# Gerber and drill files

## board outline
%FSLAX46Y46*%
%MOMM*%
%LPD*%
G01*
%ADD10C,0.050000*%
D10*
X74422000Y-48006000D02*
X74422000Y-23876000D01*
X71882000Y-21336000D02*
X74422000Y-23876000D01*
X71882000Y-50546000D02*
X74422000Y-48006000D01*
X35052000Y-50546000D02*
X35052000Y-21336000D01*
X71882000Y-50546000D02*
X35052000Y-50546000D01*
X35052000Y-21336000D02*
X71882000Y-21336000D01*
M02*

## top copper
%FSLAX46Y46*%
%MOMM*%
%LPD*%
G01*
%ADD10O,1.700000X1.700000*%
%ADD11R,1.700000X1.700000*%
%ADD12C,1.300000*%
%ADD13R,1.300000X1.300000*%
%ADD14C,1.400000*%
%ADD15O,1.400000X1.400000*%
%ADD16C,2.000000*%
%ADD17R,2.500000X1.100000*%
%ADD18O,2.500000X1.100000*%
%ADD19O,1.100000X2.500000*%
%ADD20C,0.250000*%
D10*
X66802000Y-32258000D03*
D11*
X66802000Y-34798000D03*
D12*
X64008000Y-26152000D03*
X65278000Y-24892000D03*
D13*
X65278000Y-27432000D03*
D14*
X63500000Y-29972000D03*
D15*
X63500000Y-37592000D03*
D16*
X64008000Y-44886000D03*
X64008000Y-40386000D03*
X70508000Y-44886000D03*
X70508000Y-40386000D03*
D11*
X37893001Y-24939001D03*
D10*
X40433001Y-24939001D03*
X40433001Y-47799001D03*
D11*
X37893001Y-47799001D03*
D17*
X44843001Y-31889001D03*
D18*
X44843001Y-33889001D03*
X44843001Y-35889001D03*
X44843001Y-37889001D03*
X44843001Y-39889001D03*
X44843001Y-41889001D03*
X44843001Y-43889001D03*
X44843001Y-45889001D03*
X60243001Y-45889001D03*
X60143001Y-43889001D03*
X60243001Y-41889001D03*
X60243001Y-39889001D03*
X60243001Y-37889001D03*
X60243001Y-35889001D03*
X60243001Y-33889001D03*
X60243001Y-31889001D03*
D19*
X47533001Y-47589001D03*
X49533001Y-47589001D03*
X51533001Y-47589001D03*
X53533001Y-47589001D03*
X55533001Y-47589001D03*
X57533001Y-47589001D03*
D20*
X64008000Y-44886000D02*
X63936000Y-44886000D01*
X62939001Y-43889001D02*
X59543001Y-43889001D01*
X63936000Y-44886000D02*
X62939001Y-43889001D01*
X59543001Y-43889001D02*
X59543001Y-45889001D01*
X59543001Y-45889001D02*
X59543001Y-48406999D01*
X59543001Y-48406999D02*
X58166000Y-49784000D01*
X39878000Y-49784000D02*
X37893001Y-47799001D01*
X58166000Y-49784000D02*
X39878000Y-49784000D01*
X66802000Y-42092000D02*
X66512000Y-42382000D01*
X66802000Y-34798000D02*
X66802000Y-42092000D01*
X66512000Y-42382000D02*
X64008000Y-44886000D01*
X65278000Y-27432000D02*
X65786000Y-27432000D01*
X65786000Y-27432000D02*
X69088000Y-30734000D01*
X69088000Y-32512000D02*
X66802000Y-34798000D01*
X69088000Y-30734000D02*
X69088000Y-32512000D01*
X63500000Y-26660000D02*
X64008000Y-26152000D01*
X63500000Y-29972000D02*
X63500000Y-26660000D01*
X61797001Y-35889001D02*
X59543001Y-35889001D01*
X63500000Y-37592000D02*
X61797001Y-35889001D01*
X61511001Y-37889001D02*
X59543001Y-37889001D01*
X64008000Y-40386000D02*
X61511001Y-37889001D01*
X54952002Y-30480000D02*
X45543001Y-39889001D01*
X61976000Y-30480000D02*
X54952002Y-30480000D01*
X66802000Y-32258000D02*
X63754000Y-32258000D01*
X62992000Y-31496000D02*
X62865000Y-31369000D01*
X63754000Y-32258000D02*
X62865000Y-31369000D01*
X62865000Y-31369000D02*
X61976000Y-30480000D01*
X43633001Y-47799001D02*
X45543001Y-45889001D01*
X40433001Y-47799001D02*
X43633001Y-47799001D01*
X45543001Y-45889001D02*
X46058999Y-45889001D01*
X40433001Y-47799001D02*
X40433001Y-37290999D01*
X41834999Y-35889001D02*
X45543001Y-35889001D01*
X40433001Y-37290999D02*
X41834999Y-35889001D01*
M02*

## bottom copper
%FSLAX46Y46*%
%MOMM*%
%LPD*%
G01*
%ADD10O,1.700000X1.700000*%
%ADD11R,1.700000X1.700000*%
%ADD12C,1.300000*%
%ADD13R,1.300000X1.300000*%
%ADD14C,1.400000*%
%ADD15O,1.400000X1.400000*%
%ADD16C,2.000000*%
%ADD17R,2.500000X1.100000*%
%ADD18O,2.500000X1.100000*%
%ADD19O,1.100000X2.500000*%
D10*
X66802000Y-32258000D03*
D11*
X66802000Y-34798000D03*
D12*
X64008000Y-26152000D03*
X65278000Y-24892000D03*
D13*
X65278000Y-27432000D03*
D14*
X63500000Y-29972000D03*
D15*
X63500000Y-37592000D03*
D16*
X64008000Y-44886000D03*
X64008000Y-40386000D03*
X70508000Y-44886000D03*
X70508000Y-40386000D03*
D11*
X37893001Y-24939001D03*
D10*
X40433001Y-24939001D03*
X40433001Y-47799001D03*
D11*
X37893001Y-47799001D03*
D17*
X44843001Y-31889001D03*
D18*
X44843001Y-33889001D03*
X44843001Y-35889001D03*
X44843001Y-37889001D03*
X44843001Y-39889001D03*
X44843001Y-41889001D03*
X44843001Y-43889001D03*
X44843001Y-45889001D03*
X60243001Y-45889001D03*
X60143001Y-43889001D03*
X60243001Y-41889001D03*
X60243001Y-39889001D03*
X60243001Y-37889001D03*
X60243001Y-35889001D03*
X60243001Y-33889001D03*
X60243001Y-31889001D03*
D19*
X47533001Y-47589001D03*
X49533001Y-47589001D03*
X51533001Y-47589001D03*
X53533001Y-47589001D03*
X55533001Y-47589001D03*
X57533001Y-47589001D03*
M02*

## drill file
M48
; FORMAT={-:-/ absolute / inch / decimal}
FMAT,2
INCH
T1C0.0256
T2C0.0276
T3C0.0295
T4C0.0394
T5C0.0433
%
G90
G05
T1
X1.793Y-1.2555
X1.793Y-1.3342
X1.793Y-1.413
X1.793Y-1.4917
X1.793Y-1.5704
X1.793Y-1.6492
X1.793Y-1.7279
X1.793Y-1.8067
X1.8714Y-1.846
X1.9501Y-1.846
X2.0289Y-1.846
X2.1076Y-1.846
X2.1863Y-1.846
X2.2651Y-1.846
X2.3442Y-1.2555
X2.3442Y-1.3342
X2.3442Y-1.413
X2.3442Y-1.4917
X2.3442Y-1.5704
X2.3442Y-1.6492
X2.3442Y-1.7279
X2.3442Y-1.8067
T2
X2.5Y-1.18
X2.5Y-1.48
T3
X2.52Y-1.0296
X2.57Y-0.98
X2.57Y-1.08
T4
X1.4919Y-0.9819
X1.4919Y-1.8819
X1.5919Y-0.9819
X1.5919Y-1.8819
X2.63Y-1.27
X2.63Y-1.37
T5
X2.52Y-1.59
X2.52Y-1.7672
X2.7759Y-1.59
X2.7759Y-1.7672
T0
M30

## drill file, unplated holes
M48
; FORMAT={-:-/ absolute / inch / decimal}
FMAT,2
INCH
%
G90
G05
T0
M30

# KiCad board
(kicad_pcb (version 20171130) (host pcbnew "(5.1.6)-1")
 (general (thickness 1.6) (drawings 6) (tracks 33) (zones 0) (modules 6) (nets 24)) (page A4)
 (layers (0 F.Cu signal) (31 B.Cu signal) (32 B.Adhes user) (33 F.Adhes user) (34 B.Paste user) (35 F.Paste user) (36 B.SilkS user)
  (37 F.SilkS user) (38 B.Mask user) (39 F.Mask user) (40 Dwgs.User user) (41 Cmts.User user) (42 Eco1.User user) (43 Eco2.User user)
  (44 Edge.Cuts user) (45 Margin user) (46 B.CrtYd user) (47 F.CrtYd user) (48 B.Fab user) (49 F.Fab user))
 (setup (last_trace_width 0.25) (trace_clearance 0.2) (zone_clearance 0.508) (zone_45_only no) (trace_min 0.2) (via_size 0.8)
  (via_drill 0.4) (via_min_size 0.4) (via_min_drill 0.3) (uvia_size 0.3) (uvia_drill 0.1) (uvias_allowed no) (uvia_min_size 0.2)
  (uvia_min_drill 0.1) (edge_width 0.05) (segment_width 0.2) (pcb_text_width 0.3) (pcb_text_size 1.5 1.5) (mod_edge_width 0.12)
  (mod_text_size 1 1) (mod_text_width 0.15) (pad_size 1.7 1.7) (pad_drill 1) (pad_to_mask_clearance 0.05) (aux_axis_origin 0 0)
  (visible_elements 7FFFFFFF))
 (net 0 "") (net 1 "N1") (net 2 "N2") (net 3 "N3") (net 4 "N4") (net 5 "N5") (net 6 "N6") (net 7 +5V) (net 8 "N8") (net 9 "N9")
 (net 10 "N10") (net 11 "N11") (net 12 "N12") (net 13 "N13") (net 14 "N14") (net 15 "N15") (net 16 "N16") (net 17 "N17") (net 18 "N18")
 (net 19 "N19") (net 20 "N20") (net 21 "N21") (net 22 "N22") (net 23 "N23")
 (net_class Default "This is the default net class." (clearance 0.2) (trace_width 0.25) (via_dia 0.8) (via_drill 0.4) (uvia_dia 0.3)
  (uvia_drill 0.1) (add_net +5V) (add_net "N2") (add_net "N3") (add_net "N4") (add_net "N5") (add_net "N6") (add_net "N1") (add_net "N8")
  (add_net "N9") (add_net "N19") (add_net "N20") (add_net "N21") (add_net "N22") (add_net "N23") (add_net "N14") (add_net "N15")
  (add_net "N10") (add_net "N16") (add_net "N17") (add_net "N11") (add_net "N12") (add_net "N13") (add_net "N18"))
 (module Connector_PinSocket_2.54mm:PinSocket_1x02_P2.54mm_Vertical (layer F.Cu) (at 66.802 34.798 180)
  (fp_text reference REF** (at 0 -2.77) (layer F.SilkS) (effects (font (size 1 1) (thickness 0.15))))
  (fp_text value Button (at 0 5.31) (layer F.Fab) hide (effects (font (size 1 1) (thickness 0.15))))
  (pad 2 thru_hole oval (at 0 2.54 180) (size 1.7 1.7) (drill 1) (layers *.Cu *.Mask) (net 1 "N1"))
  (pad 1 thru_hole rect (at 0 0 180) (size 1.7 1.7) (drill 1) (layers *.Cu *.Mask) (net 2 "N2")))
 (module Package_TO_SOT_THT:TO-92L (layer F.Cu) (at 65.278 27.432 90)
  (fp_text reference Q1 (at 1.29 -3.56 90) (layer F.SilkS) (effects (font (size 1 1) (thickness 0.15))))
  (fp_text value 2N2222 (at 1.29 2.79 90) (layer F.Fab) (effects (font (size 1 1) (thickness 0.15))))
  (pad 2 thru_hole circle (at 1.28 -1.27 180) (size 1.3 1.3) (drill 0.75) (layers *.Cu *.Mask) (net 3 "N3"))
  (pad 3 thru_hole circle (at 2.54 0 180) (size 1.3 1.3) (drill 0.75) (layers *.Cu *.Mask) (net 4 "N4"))
  (pad 1 thru_hole rect (at 0 0 180) (size 1.3 1.3) (drill 0.75) (layers *.Cu *.Mask) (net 2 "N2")))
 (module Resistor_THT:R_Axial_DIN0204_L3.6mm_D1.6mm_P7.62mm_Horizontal (layer F.Cu) (at 63.5 29.972 270)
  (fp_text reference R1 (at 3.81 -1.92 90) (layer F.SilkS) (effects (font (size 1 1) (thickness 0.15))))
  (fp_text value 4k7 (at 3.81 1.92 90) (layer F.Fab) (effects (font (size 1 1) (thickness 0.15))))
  (pad 1 thru_hole circle (at 0 0 270) (size 1.4 1.4) (drill 0.7) (layers *.Cu *.Mask) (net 3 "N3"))
  (pad 2 thru_hole oval (at 7.62 0 270) (size 1.4 1.4) (drill 0.7) (layers *.Cu *.Mask) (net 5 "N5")))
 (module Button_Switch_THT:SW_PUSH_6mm (layer F.Cu) (at 64.008 40.386)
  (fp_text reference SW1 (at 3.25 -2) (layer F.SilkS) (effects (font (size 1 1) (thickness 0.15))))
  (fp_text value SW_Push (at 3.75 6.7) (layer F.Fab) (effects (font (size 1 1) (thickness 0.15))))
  (pad 2 thru_hole circle (at 0 4.5 90) (size 2 2) (drill 1.1) (layers *.Cu *.Mask) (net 2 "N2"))
  (pad 1 thru_hole circle (at 0 0 90) (size 2 2) (drill 1.1) (layers *.Cu *.Mask) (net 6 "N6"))
  (pad 2 thru_hole circle (at 6.5 4.5 90) (size 2 2) (drill 1.1) (layers *.Cu *.Mask))
  (pad 1 thru_hole circle (at 6.5 0 90) (size 2 2) (drill 1.1) (layers *.Cu *.Mask)))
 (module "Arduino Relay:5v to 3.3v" (layer F.Cu) (at 39.163001 36.369001)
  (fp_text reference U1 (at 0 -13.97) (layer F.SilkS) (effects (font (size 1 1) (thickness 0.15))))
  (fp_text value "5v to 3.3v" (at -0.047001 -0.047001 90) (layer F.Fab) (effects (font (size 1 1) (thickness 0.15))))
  (pad 1 thru_hole rect (at -1.27 -11.43) (size 1.7 1.7) (drill 1) (layers *.Cu *.Mask))
  (pad 2 thru_hole oval (at 1.27 -11.43) (size 1.7 1.7) (drill 1) (layers *.Cu *.Mask) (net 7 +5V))
  (pad 3 thru_hole oval (at 1.27 11.43) (size 1.7 1.7) (drill 1) (layers *.Cu *.Mask) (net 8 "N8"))
  (pad 1 thru_hole rect (at -1.27 11.43) (size 1.7 1.7) (drill 1) (layers *.Cu *.Mask) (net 2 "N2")))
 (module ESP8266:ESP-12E (layer F.Cu) (at 45.543001 31.889001)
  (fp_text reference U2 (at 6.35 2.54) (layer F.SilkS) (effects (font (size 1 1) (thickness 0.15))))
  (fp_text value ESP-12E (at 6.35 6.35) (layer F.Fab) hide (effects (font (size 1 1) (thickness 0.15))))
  (pad 1 thru_hole rect (at 0 0) (size 2.5 1.1) (drill 0.65 (offset -0.7 0)) (layers *.Cu *.Mask F.SilkS) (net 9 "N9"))
  (pad 2 thru_hole oval (at 0 2) (size 2.5 1.1) (drill 0.65 (offset -0.7 0)) (layers *.Cu *.Mask F.SilkS) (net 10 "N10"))
  (pad 3 thru_hole oval (at 0 4) (size 2.5 1.1) (drill 0.65 (offset -0.7 0)) (layers *.Cu *.Mask F.SilkS) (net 8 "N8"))
  (pad 4 thru_hole oval (at 0 6) (size 2.5 1.1) (drill 0.65 (offset -0.7 0)) (layers *.Cu *.Mask F.SilkS) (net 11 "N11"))
  (pad 5 thru_hole oval (at 0 8) (size 2.5 1.1) (drill 0.65 (offset -0.7 0)) (layers *.Cu *.Mask F.SilkS) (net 1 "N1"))
  (pad 6 thru_hole oval (at 0 10) (size 2.5 1.1) (drill 0.65 (offset -0.7 0)) (layers *.Cu *.Mask F.SilkS) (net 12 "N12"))
  (pad 7 thru_hole oval (at 0 12) (size 2.5 1.1) (drill 0.65 (offset -0.7 0)) (layers *.Cu *.Mask F.SilkS) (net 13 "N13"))
  (pad 8 thru_hole oval (at 0 14) (size 2.5 1.1) (drill 0.65 (offset -0.7 0)) (layers *.Cu *.Mask F.SilkS) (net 8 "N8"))
  (pad 15 thru_hole oval (at 14 14) (size 2.5 1.1) (drill 0.65 (offset 0.7 0)) (layers *.Cu *.Mask F.SilkS) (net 2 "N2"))
  (pad 16 thru_hole oval (at 14 12) (size 2.5 1.1) (drill 0.65 (offset 0.6 0)) (layers *.Cu *.Mask F.SilkS) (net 2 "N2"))
  (pad 17 thru_hole oval (at 14 10) (size 2.5 1.1) (drill 0.65 (offset 0.7 0)) (layers *.Cu *.Mask F.SilkS) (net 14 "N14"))
  (pad 18 thru_hole oval (at 14 8) (size 2.5 1.1) (drill 0.65 (offset 0.7 0)) (layers *.Cu *.Mask F.SilkS) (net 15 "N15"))
  (pad 19 thru_hole oval (at 14 6) (size 2.5 1.1) (drill 0.65 (offset 0.7 0)) (layers *.Cu *.Mask F.SilkS) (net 6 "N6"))
  (pad 20 thru_hole oval (at 14 4) (size 2.5 1.1) (drill 0.65 (offset 0.7 0)) (layers *.Cu *.Mask F.SilkS) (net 5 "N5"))
  (pad 21 thru_hole oval (at 14 2) (size 2.5 1.1) (drill 0.65 (offset 0.7 0)) (layers *.Cu *.Mask F.SilkS) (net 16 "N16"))
  (pad 22 thru_hole oval (at 14 0) (size 2.5 1.1) (drill 0.65 (offset 0.7 0)) (layers *.Cu *.Mask F.SilkS) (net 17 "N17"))
  (pad 9 thru_hole oval (at 1.99 15 90) (size 2.5 1.1) (drill 0.65 (offset -0.7 0)) (layers *.Cu *.Mask F.SilkS) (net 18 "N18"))
  (pad 10 thru_hole oval (at 3.99 15 90) (size 2.5 1.1) (drill 0.65 (offset -0.7 0)) (layers *.Cu *.Mask F.SilkS) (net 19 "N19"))
  (pad 11 thru_hole oval (at 5.99 15 90) (size 2.5 1.1) (drill 0.65 (offset -0.7 0)) (layers *.Cu *.Mask F.SilkS) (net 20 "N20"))
  (pad 12 thru_hole oval (at 7.99 15 90) (size 2.5 1.1) (drill 0.65 (offset -0.7 0)) (layers *.Cu *.Mask F.SilkS) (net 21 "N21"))
  (pad 13 thru_hole oval (at 9.99 15 90) (size 2.5 1.1) (drill 0.65 (offset -0.7 0)) (layers *.Cu *.Mask F.SilkS) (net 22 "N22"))
  (pad 14 thru_hole oval (at 11.99 15 90) (size 2.5 1.1) (drill 0.65 (offset -0.7 0)) (layers *.Cu *.Mask F.SilkS) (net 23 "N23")))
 (gr_line (start 74.422 48.006) (end 74.422 23.876) (layer Edge.Cuts) (width 0.05))
 (gr_line (start 71.882 21.336) (end 74.422 23.876) (layer Edge.Cuts) (width 0.05))
 (gr_line (start 71.882 50.546) (end 74.422 48.006) (layer Edge.Cuts) (width 0.05))
 (gr_line (start 35.052 50.546) (end 35.052 21.336) (layer Edge.Cuts) (width 0.05))
 (gr_line (start 71.882 50.546) (end 35.052 50.546) (layer Edge.Cuts) (width 0.05))
 (gr_line (start 35.052 21.336) (end 71.882 21.336) (layer Edge.Cuts) (width 0.05))
 (segment (start 64.008 44.886) (end 63.936 44.886) (width 0.25) (layer F.Cu) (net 2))
 (segment (start 62.939001 43.889001) (end 59.543001 43.889001) (width 0.25) (layer F.Cu) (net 2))
 (segment (start 63.936 44.886) (end 62.939001 43.889001) (width 0.25) (layer F.Cu) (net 2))
 (segment (start 59.543001 43.889001) (end 59.543001 45.889001) (width 0.25) (layer F.Cu) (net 2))
 (segment (start 59.543001 45.889001) (end 59.543001 48.406999) (width 0.25) (layer F.Cu) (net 2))
 (segment (start 59.543001 48.406999) (end 58.166 49.784) (width 0.25) (layer F.Cu) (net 2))
 (segment (start 39.878 49.784) (end 37.893001 47.799001) (width 0.25) (layer F.Cu) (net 2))
 (segment (start 58.166 49.784) (end 39.878 49.784) (width 0.25) (layer F.Cu) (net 2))
 (segment (start 66.802 42.092) (end 66.512 42.382) (width 0.25) (layer F.Cu) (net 2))
 (segment (start 66.802 34.798) (end 66.802 42.092) (width 0.25) (layer F.Cu) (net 2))
 (segment (start 66.512 42.382) (end 64.008 44.886) (width 0.25) (layer F.Cu) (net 2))
 (segment (start 65.278 27.432) (end 65.786 27.432) (width 0.25) (layer F.Cu) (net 2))
 (segment (start 65.786 27.432) (end 69.088 30.734) (width 0.25) (layer F.Cu) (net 2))
 (segment (start 69.088 32.512) (end 66.802 34.798) (width 0.25) (layer F.Cu) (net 2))
 (segment (start 69.088 30.734) (end 69.088 32.512) (width 0.25) (layer F.Cu) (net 2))
 (segment (start 63.5 26.66) (end 64.008 26.152) (width 0.25) (layer F.Cu) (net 3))
 (segment (start 63.5 29.972) (end 63.5 26.66) (width 0.25) (layer F.Cu) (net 3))
 (segment (start 61.797001 35.889001) (end 59.543001 35.889001) (width 0.25) (layer F.Cu) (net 5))
 (segment (start 63.5 37.592) (end 61.797001 35.889001) (width 0.25) (layer F.Cu) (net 5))
 (segment (start 61.511001 37.889001) (end 59.543001 37.889001) (width 0.25) (layer F.Cu) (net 6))
 (segment (start 64.008 40.386) (end 61.511001 37.889001) (width 0.25) (layer F.Cu) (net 6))
 (segment (start 54.952002 30.48) (end 45.543001 39.889001) (width 0.25) (layer F.Cu) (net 1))
 (segment (start 61.976 30.48) (end 54.952002 30.48) (width 0.25) (layer F.Cu) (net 1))
 (segment (start 66.802 32.258) (end 63.754 32.258) (width 0.25) (layer F.Cu) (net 1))
 (segment (start 62.992 31.496) (end 62.865 31.369) (width 0.25) (layer F.Cu) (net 1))
 (segment (start 63.754 32.258) (end 62.865 31.369) (width 0.25) (layer F.Cu) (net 1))
 (segment (start 62.865 31.369) (end 61.976 30.48) (width 0.25) (layer F.Cu) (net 1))
 (segment (start 43.633001 47.799001) (end 45.543001 45.889001) (width 0.25) (layer F.Cu) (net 8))
 (segment (start 40.433001 47.799001) (end 43.633001 47.799001) (width 0.25) (layer F.Cu) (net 8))
 (segment (start 45.543001 45.889001) (end 46.058999 45.889001) (width 0.25) (layer F.Cu) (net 8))
 (segment (start 40.433001 47.799001) (end 40.433001 37.290999) (width 0.25) (layer F.Cu) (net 8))
 (segment (start 41.834999 35.889001) (end 45.543001 35.889001) (width 0.25) (layer F.Cu) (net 8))
 (segment (start 40.433001 37.290999) (end 41.834999 35.889001) (width 0.25) (layer F.Cu) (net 8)))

